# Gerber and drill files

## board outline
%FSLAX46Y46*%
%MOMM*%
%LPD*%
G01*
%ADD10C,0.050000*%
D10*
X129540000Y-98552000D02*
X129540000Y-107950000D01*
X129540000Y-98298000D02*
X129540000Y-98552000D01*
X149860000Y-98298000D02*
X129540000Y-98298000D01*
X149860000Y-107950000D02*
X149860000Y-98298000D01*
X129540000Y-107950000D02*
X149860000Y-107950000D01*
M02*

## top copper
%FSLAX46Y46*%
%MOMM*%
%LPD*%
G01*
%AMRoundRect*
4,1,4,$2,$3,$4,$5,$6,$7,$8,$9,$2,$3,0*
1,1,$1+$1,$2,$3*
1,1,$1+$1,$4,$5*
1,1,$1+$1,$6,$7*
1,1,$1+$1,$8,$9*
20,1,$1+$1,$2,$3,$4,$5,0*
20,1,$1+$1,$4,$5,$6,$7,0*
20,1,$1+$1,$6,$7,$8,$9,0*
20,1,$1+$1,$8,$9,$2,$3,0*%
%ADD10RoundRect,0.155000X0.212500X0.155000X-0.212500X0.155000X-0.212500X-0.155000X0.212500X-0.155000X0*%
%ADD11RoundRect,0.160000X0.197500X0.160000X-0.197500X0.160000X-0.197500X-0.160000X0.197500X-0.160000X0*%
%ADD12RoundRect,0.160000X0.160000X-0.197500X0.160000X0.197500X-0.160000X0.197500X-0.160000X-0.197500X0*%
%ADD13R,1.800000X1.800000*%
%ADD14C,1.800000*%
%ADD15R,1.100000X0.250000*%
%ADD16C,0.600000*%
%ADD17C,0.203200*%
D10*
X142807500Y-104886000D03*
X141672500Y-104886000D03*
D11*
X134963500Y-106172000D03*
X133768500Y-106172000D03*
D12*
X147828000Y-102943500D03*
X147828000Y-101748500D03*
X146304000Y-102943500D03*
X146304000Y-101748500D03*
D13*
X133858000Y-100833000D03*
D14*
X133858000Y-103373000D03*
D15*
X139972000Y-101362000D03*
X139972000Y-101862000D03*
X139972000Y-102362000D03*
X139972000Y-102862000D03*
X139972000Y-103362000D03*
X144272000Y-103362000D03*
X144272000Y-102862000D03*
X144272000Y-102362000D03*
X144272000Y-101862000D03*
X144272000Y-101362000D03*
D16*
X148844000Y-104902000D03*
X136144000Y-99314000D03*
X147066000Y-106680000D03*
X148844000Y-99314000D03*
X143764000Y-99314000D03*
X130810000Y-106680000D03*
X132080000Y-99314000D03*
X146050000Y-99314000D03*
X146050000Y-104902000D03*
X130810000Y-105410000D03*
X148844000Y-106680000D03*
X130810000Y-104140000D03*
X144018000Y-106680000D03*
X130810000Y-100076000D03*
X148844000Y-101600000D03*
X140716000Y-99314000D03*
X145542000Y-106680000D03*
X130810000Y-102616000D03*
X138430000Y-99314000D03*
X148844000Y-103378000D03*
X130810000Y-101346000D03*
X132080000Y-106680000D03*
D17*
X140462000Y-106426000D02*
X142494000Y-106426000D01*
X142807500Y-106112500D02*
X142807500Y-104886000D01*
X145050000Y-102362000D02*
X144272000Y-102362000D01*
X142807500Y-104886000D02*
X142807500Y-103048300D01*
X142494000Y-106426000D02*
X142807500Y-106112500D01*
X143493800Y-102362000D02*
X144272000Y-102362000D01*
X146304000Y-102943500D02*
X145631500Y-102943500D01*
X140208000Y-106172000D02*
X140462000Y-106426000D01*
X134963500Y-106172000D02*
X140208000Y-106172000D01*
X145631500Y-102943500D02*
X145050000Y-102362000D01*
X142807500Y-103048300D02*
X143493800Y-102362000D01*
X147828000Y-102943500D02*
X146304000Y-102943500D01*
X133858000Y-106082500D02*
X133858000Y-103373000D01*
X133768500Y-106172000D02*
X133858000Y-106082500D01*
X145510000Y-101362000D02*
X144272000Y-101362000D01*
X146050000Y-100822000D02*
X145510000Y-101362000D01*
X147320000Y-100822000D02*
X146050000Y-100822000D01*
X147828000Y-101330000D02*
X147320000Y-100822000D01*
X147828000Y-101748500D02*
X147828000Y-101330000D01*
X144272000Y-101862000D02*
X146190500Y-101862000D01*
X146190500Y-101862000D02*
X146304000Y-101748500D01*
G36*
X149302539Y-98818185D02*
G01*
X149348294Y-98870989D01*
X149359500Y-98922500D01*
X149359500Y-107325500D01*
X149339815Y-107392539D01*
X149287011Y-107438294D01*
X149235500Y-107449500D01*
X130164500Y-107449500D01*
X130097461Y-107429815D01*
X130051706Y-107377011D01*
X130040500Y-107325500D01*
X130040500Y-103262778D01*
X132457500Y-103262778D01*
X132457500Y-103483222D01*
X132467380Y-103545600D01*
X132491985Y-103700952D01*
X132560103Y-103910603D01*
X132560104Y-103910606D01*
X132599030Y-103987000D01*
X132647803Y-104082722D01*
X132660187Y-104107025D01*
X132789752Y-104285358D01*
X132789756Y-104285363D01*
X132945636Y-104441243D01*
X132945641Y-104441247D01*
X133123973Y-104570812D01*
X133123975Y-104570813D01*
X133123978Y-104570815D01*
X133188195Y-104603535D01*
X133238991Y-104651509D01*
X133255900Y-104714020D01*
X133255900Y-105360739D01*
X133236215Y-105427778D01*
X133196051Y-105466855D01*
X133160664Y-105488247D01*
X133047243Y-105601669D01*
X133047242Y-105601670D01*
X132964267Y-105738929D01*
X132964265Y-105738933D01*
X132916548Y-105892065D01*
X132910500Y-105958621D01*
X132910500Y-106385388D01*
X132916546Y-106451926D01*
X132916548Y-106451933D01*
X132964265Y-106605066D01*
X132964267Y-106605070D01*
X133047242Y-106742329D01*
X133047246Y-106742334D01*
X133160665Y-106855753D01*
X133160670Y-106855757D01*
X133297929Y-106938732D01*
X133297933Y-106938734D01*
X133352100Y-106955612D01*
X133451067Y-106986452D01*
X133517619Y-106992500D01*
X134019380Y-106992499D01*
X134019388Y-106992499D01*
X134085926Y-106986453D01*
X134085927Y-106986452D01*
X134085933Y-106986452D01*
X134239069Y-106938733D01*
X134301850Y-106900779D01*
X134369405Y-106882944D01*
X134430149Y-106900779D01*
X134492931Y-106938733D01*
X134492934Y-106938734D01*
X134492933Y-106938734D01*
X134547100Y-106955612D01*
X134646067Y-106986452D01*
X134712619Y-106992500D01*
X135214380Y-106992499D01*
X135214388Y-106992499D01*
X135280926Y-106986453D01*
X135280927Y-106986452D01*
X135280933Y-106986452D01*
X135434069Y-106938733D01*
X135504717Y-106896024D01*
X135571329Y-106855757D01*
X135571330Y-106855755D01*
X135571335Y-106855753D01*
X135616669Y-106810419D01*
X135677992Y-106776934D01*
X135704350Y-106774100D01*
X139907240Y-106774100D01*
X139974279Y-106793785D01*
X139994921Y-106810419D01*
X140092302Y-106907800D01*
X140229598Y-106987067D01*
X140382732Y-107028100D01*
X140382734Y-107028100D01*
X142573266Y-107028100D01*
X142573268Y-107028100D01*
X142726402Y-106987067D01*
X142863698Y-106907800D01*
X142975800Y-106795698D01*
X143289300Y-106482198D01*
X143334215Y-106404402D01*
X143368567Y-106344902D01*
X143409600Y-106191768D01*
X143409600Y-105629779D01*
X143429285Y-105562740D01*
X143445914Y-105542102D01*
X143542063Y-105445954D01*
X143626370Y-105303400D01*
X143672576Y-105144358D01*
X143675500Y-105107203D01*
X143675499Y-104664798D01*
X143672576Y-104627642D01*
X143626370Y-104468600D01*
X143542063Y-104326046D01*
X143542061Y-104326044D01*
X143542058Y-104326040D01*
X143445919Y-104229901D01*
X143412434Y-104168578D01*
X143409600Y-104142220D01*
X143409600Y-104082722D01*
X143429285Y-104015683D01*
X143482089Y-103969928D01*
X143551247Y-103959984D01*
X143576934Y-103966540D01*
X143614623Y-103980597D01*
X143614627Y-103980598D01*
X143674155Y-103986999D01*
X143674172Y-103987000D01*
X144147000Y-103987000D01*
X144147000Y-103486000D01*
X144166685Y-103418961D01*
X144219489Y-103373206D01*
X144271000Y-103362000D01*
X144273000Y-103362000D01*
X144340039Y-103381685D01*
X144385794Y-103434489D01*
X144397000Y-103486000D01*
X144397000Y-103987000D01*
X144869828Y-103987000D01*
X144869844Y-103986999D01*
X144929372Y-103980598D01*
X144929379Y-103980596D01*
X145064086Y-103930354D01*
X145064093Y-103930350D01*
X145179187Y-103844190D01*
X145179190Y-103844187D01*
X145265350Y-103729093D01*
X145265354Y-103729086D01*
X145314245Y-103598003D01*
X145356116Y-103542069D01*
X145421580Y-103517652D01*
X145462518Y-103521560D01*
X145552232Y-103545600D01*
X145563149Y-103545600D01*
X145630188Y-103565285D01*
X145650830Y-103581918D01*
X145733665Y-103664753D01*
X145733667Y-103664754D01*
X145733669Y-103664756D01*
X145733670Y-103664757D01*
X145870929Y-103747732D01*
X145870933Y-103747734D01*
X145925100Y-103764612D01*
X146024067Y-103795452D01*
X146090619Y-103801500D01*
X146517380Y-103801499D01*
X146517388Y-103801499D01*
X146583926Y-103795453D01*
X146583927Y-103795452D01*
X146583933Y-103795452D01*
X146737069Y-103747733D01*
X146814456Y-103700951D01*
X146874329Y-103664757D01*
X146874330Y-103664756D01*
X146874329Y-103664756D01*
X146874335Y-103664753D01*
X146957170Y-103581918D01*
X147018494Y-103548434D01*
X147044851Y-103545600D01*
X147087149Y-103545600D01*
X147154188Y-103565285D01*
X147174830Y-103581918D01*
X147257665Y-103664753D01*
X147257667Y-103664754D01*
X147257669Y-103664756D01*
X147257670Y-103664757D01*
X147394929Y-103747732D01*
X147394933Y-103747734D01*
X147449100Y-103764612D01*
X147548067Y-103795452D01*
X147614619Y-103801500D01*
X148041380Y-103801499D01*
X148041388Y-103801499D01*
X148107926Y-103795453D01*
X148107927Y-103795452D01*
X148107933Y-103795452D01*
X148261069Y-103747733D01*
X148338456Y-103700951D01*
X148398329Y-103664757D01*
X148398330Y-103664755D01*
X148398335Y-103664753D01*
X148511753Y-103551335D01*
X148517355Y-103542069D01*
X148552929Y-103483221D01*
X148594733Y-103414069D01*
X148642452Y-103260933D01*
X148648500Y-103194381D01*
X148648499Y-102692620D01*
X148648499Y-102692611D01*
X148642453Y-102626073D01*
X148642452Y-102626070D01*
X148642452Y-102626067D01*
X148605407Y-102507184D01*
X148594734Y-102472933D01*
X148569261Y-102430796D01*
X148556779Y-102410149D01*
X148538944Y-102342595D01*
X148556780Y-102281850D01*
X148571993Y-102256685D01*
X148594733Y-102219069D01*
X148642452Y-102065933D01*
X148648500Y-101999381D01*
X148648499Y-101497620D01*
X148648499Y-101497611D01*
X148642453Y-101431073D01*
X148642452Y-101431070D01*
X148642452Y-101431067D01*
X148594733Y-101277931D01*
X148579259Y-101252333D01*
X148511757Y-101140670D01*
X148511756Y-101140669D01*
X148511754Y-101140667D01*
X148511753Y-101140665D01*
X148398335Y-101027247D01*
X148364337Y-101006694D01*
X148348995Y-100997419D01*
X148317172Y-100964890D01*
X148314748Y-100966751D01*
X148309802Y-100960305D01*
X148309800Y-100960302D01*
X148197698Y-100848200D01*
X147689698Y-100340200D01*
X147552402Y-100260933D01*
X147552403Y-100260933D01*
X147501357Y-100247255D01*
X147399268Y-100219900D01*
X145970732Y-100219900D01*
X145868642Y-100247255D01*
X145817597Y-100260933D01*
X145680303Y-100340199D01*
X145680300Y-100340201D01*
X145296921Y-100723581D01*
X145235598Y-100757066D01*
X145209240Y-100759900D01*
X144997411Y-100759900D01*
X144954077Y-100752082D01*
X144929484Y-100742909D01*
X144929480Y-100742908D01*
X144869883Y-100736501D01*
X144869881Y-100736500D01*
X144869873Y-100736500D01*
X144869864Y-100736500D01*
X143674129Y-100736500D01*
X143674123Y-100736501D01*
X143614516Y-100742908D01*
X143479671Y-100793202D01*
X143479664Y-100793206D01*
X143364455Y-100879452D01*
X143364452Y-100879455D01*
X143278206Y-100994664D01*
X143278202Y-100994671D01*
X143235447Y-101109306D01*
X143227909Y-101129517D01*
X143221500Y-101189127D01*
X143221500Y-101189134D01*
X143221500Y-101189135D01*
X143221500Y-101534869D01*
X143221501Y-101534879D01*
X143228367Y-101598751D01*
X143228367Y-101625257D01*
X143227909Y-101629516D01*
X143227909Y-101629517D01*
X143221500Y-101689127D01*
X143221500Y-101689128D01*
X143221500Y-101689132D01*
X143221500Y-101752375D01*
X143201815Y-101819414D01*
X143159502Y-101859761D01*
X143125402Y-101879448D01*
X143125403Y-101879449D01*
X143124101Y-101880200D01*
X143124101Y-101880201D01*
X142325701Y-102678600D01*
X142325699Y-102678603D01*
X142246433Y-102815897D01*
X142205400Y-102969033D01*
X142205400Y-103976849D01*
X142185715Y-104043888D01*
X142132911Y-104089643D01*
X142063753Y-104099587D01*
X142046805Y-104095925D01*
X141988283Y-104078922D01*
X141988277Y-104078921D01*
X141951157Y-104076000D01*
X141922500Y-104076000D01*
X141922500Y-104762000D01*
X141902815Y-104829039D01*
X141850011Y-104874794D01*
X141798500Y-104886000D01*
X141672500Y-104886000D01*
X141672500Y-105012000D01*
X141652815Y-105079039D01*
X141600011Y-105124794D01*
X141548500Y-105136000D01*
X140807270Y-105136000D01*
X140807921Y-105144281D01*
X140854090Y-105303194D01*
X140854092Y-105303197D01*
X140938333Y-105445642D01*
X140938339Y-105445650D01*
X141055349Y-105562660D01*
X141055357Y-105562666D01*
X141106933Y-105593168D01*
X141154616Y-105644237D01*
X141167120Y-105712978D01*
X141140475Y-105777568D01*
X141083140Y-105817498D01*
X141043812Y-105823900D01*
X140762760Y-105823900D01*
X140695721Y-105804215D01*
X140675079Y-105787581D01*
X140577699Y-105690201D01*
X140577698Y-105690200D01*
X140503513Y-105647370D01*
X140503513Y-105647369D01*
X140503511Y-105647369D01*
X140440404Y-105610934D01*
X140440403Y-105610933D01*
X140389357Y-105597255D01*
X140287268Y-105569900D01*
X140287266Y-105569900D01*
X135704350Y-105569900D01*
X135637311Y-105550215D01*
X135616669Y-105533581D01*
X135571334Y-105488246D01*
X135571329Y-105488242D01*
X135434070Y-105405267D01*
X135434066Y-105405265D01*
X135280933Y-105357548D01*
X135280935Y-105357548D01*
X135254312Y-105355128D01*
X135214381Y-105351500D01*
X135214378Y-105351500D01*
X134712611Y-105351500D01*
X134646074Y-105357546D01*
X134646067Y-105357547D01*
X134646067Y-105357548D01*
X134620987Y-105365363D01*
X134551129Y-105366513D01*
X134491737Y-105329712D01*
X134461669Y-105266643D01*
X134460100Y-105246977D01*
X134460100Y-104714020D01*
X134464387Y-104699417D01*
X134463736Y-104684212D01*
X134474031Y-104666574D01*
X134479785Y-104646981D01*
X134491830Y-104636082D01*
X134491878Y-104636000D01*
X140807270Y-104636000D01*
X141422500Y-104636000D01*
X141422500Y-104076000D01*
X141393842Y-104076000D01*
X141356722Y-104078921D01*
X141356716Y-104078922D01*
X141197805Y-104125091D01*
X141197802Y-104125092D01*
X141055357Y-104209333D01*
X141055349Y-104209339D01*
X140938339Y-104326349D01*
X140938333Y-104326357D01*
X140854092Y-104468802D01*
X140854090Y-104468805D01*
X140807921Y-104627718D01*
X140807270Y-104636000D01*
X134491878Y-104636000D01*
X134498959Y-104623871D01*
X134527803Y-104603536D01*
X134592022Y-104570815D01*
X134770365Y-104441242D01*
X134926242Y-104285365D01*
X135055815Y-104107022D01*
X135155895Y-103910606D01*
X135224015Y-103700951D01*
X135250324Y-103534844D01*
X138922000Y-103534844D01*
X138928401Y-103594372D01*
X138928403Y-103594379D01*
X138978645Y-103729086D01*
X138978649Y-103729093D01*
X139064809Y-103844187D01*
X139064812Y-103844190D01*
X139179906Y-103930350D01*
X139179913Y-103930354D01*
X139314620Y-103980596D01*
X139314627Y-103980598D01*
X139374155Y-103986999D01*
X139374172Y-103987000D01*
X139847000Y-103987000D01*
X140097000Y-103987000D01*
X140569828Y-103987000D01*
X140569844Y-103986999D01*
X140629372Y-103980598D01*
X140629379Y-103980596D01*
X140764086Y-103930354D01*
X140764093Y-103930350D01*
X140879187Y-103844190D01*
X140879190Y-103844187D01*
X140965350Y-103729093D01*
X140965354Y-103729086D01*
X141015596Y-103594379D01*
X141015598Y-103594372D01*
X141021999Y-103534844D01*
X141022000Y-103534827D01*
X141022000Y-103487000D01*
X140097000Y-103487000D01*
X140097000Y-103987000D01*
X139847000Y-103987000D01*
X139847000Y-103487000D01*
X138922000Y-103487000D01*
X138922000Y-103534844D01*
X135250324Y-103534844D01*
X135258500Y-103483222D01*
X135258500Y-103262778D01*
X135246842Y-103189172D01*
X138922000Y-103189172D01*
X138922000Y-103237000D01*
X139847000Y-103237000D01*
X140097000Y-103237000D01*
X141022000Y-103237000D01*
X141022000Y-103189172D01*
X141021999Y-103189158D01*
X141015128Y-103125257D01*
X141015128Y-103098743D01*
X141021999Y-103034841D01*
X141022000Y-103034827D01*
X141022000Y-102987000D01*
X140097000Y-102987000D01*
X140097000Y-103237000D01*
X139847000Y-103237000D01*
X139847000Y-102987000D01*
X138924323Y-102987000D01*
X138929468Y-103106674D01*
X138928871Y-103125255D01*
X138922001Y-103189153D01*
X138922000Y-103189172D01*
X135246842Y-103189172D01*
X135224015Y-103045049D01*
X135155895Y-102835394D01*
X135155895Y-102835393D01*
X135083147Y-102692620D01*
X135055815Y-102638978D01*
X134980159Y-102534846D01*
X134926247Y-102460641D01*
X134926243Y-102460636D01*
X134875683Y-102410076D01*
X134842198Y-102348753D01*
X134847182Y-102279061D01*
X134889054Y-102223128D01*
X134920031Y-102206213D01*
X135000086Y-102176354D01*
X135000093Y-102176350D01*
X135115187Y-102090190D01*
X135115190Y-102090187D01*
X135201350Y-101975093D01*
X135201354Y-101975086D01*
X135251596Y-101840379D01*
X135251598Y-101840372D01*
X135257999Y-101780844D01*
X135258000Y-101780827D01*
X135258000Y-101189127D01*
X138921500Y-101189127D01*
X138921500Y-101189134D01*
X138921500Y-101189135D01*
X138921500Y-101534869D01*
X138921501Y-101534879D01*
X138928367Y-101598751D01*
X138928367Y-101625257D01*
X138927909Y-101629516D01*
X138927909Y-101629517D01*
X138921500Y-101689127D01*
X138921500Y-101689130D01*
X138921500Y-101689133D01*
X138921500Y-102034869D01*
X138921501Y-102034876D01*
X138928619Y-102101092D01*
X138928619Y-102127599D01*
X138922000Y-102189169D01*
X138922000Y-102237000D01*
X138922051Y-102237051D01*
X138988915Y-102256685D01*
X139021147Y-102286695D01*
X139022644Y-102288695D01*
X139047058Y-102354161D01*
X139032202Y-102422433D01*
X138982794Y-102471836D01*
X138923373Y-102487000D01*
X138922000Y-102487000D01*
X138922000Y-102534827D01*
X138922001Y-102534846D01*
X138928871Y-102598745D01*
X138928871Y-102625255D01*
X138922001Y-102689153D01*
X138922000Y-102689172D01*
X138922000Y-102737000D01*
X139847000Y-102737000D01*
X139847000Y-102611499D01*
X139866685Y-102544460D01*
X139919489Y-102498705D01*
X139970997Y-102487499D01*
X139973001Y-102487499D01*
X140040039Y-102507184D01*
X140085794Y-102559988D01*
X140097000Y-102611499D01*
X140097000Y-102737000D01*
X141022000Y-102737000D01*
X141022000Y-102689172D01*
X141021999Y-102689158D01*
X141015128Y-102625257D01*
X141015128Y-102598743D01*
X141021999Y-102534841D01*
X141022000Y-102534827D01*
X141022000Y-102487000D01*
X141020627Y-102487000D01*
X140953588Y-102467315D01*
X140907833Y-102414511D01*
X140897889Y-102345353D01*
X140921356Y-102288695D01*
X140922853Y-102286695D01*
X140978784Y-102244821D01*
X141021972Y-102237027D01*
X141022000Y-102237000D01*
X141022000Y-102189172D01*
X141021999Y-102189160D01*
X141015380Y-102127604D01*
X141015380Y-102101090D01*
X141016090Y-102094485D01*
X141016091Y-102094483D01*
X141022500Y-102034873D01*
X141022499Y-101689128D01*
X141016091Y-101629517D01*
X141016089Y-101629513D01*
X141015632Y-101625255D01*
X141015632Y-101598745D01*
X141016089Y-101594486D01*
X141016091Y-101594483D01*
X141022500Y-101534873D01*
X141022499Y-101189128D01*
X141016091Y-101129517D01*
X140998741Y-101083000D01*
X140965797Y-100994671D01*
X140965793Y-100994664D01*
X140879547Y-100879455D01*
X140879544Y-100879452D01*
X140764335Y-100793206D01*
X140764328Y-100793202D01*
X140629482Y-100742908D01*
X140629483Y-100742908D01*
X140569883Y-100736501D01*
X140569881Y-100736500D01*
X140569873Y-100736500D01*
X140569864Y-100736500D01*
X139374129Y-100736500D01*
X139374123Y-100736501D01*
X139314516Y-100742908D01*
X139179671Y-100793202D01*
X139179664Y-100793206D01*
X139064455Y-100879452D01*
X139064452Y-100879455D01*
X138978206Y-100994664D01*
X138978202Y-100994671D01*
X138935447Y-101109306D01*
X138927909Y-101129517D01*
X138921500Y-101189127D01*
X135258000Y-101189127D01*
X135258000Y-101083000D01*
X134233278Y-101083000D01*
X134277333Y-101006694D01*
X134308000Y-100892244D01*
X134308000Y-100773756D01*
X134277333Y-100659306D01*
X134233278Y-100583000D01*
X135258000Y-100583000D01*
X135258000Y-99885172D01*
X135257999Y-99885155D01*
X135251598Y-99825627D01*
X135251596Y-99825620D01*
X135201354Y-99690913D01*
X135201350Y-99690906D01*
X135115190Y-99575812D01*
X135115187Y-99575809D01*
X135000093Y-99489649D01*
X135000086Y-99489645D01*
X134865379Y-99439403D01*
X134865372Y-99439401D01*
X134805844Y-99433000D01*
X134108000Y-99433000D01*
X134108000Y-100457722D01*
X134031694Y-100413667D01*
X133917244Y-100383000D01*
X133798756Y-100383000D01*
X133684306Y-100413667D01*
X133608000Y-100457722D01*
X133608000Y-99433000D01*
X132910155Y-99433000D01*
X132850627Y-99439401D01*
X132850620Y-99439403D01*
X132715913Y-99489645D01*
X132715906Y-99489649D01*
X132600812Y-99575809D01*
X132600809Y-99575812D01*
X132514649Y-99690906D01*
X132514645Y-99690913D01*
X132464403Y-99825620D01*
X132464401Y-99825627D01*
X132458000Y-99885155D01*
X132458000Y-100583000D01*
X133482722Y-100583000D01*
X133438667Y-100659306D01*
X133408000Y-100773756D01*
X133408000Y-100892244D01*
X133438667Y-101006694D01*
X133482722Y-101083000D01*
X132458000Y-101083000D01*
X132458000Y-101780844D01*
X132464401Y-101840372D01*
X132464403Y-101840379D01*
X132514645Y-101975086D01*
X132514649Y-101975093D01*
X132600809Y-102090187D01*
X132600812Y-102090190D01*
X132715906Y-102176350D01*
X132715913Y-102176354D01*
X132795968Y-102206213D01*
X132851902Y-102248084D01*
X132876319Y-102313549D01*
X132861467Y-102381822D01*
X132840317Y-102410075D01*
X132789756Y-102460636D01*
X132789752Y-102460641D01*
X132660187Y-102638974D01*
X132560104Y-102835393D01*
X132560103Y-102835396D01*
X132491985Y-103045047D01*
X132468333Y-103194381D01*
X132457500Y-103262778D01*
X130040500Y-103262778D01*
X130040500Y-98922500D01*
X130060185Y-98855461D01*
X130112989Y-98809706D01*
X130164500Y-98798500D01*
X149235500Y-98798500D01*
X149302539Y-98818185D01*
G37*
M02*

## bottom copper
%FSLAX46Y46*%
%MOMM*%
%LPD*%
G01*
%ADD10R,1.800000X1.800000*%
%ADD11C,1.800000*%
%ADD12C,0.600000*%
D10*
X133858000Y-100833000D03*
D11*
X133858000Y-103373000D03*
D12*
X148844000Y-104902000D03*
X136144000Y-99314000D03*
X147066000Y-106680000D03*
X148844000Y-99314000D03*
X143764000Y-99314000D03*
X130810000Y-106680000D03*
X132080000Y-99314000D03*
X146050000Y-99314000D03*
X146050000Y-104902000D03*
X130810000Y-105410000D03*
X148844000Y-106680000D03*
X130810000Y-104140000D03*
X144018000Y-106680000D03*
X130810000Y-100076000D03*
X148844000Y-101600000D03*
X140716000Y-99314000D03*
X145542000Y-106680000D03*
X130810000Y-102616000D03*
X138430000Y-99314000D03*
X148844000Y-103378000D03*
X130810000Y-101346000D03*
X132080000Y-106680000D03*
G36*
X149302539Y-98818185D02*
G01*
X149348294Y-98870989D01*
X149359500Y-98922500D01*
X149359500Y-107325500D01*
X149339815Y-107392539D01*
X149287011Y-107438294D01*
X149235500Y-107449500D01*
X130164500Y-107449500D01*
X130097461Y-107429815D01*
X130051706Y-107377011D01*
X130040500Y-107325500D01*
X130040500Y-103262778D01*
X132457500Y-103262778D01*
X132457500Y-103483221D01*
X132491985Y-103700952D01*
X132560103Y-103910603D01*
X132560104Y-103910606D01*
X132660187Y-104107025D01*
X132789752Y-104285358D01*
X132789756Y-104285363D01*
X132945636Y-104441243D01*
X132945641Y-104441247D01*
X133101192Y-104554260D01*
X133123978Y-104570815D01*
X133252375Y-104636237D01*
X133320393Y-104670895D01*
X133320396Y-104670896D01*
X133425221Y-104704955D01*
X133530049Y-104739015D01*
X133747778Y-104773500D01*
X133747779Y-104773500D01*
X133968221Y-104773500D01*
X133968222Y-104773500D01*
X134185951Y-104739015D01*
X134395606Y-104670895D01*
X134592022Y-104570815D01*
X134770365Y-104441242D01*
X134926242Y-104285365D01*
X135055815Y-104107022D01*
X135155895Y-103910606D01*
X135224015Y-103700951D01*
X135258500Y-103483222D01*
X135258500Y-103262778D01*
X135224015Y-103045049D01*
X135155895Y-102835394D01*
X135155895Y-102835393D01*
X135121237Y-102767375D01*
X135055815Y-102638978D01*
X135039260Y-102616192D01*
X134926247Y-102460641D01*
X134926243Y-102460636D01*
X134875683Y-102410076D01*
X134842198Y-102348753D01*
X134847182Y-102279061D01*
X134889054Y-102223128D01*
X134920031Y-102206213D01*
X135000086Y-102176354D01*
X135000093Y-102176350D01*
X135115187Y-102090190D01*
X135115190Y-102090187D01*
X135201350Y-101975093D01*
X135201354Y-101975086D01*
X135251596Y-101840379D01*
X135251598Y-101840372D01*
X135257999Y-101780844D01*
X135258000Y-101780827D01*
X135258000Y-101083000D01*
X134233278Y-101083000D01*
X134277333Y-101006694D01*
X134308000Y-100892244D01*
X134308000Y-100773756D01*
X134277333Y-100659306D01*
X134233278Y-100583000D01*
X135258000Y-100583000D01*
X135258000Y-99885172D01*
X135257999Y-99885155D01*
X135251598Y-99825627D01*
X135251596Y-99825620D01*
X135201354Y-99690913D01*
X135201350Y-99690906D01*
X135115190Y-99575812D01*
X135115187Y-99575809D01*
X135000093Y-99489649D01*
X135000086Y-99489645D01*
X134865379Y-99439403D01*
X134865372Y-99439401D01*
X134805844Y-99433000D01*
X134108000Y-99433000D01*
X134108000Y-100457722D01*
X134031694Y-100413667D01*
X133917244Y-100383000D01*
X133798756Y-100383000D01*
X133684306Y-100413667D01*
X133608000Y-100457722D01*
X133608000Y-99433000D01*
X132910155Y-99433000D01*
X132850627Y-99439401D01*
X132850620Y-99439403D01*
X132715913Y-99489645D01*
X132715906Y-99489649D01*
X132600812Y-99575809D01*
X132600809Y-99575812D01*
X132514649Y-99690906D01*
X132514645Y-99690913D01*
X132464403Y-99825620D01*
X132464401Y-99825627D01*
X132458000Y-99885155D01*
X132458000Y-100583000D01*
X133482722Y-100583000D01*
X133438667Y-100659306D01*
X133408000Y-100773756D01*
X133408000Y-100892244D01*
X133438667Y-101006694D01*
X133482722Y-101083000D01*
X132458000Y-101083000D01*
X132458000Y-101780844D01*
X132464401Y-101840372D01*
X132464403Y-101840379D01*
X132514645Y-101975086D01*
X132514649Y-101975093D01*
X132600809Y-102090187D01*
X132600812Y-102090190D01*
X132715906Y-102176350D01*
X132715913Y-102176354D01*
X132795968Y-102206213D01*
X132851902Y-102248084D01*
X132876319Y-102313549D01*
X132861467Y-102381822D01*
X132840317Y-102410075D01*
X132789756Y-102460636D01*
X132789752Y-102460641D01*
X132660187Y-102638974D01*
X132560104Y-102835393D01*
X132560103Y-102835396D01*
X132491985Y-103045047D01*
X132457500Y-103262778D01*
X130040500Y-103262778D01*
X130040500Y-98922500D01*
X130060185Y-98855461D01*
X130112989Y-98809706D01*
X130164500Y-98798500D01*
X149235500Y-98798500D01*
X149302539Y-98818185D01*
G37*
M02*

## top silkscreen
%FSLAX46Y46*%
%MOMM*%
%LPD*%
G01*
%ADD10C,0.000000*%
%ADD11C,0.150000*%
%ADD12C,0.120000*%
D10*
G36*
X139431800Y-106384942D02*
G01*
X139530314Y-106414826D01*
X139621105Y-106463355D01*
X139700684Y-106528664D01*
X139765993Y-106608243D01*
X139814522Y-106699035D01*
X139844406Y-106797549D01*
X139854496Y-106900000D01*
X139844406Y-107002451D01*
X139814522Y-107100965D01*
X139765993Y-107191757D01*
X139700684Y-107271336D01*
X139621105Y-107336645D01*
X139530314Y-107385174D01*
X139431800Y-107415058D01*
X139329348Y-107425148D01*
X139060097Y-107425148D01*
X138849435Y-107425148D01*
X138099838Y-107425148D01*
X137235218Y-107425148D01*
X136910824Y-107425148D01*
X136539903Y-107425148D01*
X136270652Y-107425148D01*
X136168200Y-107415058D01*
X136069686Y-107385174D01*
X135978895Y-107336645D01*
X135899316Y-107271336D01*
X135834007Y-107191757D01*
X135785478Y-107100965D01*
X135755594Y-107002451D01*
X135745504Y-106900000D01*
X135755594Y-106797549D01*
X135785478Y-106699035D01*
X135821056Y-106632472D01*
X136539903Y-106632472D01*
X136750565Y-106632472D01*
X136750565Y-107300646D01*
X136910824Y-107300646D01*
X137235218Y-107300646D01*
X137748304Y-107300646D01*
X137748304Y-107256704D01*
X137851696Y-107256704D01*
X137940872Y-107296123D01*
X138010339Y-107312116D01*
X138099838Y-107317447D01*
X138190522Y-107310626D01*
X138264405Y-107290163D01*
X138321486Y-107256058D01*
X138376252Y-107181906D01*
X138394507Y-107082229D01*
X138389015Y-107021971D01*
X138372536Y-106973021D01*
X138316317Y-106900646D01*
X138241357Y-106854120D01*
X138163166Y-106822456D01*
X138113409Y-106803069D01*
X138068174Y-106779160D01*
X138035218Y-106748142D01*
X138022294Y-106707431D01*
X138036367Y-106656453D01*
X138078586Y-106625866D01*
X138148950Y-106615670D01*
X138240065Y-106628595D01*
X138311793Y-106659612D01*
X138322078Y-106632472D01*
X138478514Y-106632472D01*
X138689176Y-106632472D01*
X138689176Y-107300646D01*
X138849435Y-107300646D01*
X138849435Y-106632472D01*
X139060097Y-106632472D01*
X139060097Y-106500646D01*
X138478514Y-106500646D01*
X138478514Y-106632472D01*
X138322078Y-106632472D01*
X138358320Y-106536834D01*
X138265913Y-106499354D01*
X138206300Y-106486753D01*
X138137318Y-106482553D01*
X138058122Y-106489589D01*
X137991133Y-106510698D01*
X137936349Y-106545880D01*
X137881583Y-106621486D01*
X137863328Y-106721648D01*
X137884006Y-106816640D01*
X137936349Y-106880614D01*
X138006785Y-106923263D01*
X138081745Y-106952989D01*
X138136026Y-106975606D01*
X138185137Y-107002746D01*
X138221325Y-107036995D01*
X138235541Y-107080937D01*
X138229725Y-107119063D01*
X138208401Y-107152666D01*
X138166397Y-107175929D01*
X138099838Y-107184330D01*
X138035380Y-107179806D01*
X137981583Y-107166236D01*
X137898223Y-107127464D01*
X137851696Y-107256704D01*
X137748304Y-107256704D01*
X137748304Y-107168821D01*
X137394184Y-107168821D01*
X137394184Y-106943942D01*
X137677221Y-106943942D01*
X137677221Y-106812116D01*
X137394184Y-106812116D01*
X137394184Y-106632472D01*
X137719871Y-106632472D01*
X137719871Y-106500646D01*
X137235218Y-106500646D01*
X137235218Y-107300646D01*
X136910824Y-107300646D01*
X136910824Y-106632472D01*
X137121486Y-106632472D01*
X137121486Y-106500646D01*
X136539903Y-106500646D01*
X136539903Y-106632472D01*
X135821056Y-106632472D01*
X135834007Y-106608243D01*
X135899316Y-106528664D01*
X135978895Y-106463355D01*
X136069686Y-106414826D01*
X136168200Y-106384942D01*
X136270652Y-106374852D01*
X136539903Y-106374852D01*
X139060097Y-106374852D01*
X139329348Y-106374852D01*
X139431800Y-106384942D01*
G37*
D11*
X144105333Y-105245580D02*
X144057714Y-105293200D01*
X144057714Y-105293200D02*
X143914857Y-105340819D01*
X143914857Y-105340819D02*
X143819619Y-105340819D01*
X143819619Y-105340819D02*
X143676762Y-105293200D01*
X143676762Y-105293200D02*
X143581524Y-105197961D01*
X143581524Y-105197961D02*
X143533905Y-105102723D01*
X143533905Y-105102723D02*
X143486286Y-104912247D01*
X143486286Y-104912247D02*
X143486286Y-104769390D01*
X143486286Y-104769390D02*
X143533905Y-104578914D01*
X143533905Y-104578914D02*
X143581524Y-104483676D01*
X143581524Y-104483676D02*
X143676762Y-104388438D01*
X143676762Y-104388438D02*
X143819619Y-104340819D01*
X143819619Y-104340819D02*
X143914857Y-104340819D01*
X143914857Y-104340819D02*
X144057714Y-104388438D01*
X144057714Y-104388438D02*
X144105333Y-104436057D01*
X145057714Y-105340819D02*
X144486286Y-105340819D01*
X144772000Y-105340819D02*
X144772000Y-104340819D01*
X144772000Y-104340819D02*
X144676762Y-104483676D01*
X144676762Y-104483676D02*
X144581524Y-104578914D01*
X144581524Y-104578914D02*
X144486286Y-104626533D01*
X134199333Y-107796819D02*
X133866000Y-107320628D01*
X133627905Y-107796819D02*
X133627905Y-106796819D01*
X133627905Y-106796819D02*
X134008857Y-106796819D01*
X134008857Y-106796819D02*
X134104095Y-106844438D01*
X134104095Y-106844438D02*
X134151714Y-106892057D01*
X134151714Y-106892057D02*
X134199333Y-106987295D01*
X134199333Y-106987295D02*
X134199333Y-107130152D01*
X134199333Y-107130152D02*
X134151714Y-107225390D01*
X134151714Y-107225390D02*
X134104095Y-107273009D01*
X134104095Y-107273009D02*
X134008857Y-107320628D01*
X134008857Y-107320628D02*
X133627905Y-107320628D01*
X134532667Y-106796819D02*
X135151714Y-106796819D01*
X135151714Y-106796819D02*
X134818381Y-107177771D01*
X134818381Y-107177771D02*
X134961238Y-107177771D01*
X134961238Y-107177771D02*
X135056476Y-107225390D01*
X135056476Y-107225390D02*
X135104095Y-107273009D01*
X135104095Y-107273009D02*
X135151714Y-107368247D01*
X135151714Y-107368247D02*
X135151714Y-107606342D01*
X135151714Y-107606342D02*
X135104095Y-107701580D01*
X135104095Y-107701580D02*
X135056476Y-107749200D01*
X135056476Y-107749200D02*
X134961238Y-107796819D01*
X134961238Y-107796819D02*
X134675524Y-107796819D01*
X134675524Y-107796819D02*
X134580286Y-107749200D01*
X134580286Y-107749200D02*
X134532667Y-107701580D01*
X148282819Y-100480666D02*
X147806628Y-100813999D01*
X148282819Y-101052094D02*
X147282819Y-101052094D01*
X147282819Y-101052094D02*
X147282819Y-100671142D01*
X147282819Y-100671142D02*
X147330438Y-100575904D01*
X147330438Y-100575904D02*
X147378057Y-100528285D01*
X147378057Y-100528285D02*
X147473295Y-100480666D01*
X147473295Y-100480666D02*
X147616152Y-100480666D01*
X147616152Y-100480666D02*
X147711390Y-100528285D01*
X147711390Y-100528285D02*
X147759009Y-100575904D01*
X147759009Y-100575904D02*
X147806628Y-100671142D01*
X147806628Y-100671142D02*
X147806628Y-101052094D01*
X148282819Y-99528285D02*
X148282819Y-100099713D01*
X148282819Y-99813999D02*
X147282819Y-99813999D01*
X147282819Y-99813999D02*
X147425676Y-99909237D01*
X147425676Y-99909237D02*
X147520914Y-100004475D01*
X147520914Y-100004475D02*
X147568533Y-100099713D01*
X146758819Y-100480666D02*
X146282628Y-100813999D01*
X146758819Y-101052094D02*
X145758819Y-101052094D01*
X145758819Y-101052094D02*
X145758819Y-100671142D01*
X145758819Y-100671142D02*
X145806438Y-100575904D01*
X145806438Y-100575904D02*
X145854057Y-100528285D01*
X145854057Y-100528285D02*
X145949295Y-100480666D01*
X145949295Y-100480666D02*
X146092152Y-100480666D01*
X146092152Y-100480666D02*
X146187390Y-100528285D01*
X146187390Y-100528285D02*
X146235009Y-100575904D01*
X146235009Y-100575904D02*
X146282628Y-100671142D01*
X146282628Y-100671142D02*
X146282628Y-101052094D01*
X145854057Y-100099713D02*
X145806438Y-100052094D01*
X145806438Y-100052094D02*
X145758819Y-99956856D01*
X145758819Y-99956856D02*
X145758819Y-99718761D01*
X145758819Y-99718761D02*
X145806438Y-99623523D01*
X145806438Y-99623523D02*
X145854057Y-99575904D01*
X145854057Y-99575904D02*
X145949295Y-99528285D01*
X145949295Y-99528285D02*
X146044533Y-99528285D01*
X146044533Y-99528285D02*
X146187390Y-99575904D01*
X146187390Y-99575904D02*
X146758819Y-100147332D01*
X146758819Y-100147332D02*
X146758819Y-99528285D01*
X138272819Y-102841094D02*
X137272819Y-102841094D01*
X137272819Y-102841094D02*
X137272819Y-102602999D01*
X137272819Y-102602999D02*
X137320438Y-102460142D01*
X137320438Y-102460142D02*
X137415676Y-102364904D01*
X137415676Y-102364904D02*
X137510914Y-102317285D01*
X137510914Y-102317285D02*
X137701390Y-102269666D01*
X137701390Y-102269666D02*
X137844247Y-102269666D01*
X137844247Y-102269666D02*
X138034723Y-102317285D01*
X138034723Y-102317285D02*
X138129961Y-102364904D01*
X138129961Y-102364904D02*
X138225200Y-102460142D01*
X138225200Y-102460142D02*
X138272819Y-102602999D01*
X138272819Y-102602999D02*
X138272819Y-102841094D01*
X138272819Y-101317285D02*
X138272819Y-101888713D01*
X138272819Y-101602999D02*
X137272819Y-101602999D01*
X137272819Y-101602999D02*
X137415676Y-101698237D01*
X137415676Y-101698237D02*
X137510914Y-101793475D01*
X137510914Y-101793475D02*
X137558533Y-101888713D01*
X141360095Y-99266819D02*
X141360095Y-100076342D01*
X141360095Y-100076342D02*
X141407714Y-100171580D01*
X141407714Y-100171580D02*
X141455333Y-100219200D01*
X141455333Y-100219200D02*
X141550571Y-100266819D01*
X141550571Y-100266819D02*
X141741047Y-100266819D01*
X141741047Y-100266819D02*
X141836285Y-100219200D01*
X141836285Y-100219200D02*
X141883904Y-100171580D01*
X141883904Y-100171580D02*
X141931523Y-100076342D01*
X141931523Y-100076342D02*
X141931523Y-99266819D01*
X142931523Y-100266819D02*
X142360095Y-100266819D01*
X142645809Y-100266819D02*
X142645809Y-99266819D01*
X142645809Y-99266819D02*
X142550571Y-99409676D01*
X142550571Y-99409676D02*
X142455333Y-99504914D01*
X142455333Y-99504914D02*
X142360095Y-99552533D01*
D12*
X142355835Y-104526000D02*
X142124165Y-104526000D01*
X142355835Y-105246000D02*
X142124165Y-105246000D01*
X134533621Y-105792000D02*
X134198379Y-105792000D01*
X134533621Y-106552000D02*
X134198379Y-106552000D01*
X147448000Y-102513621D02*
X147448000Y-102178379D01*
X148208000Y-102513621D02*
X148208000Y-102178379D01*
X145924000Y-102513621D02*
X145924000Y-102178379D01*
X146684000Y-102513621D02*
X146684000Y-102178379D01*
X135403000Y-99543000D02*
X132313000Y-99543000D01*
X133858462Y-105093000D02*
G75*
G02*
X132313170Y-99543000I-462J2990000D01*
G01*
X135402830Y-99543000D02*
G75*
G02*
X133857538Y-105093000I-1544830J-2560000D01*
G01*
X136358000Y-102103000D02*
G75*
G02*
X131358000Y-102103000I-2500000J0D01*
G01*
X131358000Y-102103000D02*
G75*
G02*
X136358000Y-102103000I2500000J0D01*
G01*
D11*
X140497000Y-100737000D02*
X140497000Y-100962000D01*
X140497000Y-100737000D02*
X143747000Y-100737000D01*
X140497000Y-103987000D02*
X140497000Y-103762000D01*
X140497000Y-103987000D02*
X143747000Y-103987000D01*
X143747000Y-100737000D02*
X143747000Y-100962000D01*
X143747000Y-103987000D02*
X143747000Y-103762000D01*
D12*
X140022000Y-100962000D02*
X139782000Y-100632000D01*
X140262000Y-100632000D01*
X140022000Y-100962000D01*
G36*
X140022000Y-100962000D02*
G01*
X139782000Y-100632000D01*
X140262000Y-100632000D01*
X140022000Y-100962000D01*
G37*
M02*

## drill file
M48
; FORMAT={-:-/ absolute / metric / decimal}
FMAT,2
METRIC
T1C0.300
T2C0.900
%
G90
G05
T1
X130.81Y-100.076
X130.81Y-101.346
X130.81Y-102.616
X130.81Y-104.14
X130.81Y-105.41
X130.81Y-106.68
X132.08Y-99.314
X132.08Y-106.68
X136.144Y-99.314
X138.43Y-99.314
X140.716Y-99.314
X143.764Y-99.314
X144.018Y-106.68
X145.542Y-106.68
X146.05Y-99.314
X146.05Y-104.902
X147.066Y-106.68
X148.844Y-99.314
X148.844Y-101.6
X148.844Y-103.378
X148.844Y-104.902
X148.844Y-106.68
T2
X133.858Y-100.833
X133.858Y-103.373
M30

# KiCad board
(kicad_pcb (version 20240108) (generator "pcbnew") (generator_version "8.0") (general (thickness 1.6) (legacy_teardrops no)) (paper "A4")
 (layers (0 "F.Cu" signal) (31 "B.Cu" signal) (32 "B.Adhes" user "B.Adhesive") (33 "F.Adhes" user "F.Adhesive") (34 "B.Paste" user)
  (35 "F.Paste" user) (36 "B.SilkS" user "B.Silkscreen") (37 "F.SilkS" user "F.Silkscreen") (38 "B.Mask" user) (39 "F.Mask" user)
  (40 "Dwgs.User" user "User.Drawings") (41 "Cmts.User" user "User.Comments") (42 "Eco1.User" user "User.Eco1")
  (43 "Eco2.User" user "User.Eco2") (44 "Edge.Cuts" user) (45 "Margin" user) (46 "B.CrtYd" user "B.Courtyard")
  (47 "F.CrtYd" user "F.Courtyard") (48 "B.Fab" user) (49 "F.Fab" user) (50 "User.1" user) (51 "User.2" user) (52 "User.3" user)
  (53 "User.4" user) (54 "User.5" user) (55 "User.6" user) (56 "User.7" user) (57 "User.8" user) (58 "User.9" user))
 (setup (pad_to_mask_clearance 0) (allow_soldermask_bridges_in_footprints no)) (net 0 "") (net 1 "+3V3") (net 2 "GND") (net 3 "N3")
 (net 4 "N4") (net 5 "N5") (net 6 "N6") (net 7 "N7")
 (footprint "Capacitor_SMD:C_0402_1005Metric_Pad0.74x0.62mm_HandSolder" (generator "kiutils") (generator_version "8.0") (layer "F.Cu")
  (at 142.24 104.886 180)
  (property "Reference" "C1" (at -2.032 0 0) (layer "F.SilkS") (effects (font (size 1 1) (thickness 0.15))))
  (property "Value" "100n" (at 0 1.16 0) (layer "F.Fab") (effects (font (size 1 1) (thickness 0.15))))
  (fp_line (start -0.115835 0.36) (end 0.115835 0.36) (stroke (width 0.12) (type solid)) (layer "F.SilkS"))
  (fp_line (start -0.115835 -0.36) (end 0.115835 -0.36) (stroke (width 0.12) (type solid)) (layer "F.SilkS"))
  (pad "1" smd roundrect (at -0.5675 0 180) (size 0.735 0.62) (layers "F.Cu" "F.Paste" "F.Mask") (roundrect_rratio 0.25) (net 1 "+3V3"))
  (pad "2" smd roundrect (at 0.5675 0 180) (size 0.735 0.62) (layers "F.Cu" "F.Paste" "F.Mask") (roundrect_rratio 0.25) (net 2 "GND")))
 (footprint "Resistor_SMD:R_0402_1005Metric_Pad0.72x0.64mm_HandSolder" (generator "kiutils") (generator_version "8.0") (layer "F.Cu")
  (at 134.366 106.172 180)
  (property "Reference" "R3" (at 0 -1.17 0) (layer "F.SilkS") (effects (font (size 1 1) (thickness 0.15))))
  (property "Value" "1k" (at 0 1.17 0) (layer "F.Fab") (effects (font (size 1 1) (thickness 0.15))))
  (fp_line (start -0.167621 0.38) (end 0.167621 0.38) (stroke (width 0.12) (type solid)) (layer "F.SilkS"))
  (fp_line (start -0.167621 -0.38) (end 0.167621 -0.38) (stroke (width 0.12) (type solid)) (layer "F.SilkS"))
  (pad "1" smd roundrect (at -0.5975 0 180) (size 0.715 0.64) (layers "F.Cu" "F.Paste" "F.Mask") (roundrect_rratio 0.25) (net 1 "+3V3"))
  (pad "2" smd roundrect (at 0.5975 0 180) (size 0.715 0.64) (layers "F.Cu" "F.Paste" "F.Mask") (roundrect_rratio 0.25) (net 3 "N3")))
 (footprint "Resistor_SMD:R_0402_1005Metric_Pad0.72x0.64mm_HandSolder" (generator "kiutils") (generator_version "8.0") (layer "F.Cu")
  (at 147.828 102.346 90)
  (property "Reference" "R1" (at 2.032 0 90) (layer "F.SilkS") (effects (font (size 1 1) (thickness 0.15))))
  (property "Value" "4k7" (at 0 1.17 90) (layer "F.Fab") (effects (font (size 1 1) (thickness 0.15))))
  (fp_line (start -0.167621 -0.38) (end 0.167621 -0.38) (stroke (width 0.12) (type solid)) (layer "F.SilkS"))
  (fp_line (start -0.167621 0.38) (end 0.167621 0.38) (stroke (width 0.12) (type solid)) (layer "F.SilkS"))
  (pad "1" smd roundrect (at -0.5975 0 90) (size 0.715 0.64) (layers "F.Cu" "F.Paste" "F.Mask") (roundrect_rratio 0.25) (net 1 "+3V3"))
  (pad "2" smd roundrect (at 0.5975 0 90) (size 0.715 0.64) (layers "F.Cu" "F.Paste" "F.Mask") (roundrect_rratio 0.25) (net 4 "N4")))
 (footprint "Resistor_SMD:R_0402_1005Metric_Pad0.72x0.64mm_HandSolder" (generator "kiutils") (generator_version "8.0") (layer "F.Cu")
  (at 146.304 102.346 90)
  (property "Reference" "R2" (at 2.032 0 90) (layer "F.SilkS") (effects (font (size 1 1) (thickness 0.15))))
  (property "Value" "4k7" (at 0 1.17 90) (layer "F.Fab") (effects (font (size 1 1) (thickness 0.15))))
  (fp_line (start -0.167621 -0.38) (end 0.167621 -0.38) (stroke (width 0.12) (type solid)) (layer "F.SilkS"))
  (fp_line (start -0.167621 0.38) (end 0.167621 0.38) (stroke (width 0.12) (type solid)) (layer "F.SilkS"))
  (pad "1" smd roundrect (at -0.5975 0 90) (size 0.715 0.64) (layers "F.Cu" "F.Paste" "F.Mask") (roundrect_rratio 0.25) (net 1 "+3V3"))
  (pad "2" smd roundrect (at 0.5975 0 90) (size 0.715 0.64) (layers "F.Cu" "F.Paste" "F.Mask") (roundrect_rratio 0.25) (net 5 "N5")))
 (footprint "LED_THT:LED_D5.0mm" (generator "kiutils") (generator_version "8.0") (layer "F.Cu") (at 133.858 100.833 -90)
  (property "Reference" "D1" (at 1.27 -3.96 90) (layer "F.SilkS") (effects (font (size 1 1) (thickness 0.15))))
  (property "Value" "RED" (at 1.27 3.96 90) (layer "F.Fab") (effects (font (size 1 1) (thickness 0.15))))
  (fp_line (start -1.29 -1.545) (end -1.29 1.545) (stroke (width 0.12) (type solid)) (layer "F.SilkS"))
  (fp_arc (start 4.26 -0.000462) (mid 2.072002 2.880433) (end -1.29 1.54483) (stroke (width 0.12) (type solid)) (layer "F.SilkS"))
  (fp_arc (start -1.29 -1.54483) (mid 2.072002 -2.880433) (end 4.26 0.000462) (stroke (width 0.12) (type solid)) (layer "F.SilkS"))
  (fp_circle (center 1.27 0) (end 3.77 0) (stroke (width 0.12) (type solid)) (fill none) (layer "F.SilkS"))
  (pad "1" thru_hole rect (at 0 0 270) (size 1.8 1.8) (drill 0.9) (layers "*.Cu" "*.Mask") (remove_unused_layers no) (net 2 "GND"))
  (pad "2" thru_hole circle (at 2.54 0 270) (size 1.8 1.8) (drill 0.9) (layers "*.Cu" "*.Mask") (remove_unused_layers no) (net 3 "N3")))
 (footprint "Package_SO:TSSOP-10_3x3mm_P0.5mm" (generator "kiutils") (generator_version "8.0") (layer "F.Cu") (at 142.122 102.362)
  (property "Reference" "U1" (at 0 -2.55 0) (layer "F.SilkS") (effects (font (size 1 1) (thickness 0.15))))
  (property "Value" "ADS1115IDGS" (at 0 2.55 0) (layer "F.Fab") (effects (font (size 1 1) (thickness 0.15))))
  (fp_line (start -1.625 -1.625) (end -1.625 -1.4) (stroke (width 0.15) (type solid)) (layer "F.SilkS"))
  (fp_line (start -1.625 -1.625) (end 1.625 -1.625) (stroke (width 0.15) (type solid)) (layer "F.SilkS"))
  (fp_line (start -1.625 1.625) (end -1.625 1.4) (stroke (width 0.15) (type solid)) (layer "F.SilkS"))
  (fp_line (start -1.625 1.625) (end 1.625 1.625) (stroke (width 0.15) (type solid)) (layer "F.SilkS"))
  (fp_line (start 1.625 -1.625) (end 1.625 -1.4) (stroke (width 0.15) (type solid)) (layer "F.SilkS"))
  (fp_line (start 1.625 1.625) (end 1.625 1.4) (stroke (width 0.15) (type solid)) (layer "F.SilkS"))
  (fp_poly
   (pts (xy -2.1 -1.4) (xy -2.34 -1.73) (xy -1.86 -1.73) (xy -2.1 -1.4)) (stroke (width 0.12) (type solid)) (fill solid) (layer "F.SilkS"))
  (pad "1" smd rect (at -2.15 -1) (size 1.1 0.25) (layers "F.Cu" "F.Paste" "F.Mask") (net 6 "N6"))
  (pad "2" smd rect (at -2.15 -0.5) (size 1.1 0.25) (layers "F.Cu" "F.Paste" "F.Mask") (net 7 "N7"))
  (pad "3" smd rect (at -2.15 0) (size 1.1 0.25) (layers "F.Cu" "F.Paste" "F.Mask") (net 2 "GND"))
  (pad "4" smd rect (at -2.15 0.5) (size 1.1 0.25) (layers "F.Cu" "F.Paste" "F.Mask") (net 2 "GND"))
  (pad "5" smd rect (at -2.15 1) (size 1.1 0.25) (layers "F.Cu" "F.Paste" "F.Mask") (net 2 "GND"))
  (pad "6" smd rect (at 2.15 1) (size 1.1 0.25) (layers "F.Cu" "F.Paste" "F.Mask") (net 2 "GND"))
  (pad "7" smd rect (at 2.15 0.5) (size 1.1 0.25) (layers "F.Cu" "F.Paste" "F.Mask") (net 2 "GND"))
  (pad "8" smd rect (at 2.15 0) (size 1.1 0.25) (layers "F.Cu" "F.Paste" "F.Mask") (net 1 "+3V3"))
  (pad "9" smd rect (at 2.15 -0.5) (size 1.1 0.25) (layers "F.Cu" "F.Paste" "F.Mask") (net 5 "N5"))
  (pad "10" smd rect (at 2.15 -1) (size 1.1 0.25) (layers "F.Cu" "F.Paste" "F.Mask") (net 4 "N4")))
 (gr_line (start 129.54 98.552) (end 129.54 107.95) (stroke (width 0.05) (type default)) (layer "Edge.Cuts"))
 (gr_line (start 129.54 98.298) (end 129.54 98.552) (stroke (width 0.05) (type default)) (layer "Edge.Cuts"))
 (gr_line (start 149.86 98.298) (end 129.54 98.298) (stroke (width 0.05) (type default)) (layer "Edge.Cuts"))
 (gr_line (start 149.86 107.95) (end 149.86 98.298) (stroke (width 0.05) (type default)) (layer "Edge.Cuts"))
 (gr_line (start 129.54 107.95) (end 149.86 107.95) (stroke (width 0.05) (type default)) (layer "Edge.Cuts"))
 (gr_poly
  (pts (xy 136.539903 106.374852) (xy 136.270652 106.374852) (xy 136.1682 106.384942) (xy 136.069686 106.414826) (xy 135.978895 106.463355)
   (xy 135.899316 106.528664) (xy 135.834007 106.608243) (xy 135.785478 106.699035) (xy 135.755594 106.797549) (xy 135.745504 106.9)
   (xy 135.755594 107.002451) (xy 135.785478 107.100965) (xy 135.834007 107.191757) (xy 135.899316 107.271336) (xy 135.978895 107.336645)
   (xy 136.069686 107.385174) (xy 136.1682 107.415058) (xy 136.270652 107.425148) (xy 136.539903 107.425148) (xy 136.910824 107.425148)
   (xy 136.910824 107.300646) (xy 136.750565 107.300646) (xy 136.750565 106.632472) (xy 136.539903 106.632472) (xy 136.539903 106.500646)
   (xy 137.121486 106.500646) (xy 137.121486 106.632472) (xy 136.910824 106.632472) (xy 136.910824 107.300646) (xy 136.910824 107.425148)
   (xy 137.235218 107.425148) (xy 137.235218 107.300646) (xy 137.235218 106.500646) (xy 137.719871 106.500646) (xy 137.719871 106.632472)
   (xy 137.394184 106.632472) (xy 137.394184 106.812116) (xy 137.677221 106.812116) (xy 137.677221 106.943942) (xy 137.394184 106.943942)
   (xy 137.394184 107.168821) (xy 137.748304 107.168821) (xy 137.748304 107.300646) (xy 137.235218 107.300646) (xy 137.235218 107.425148)
   (xy 138.099838 107.425148) (xy 138.099838 107.317447) (xy 138.010339 107.312116) (xy 137.940872 107.296123) (xy 137.851696 107.256704)
   (xy 137.898223 107.127464) (xy 137.981583 107.166236) (xy 138.03538 107.179806) (xy 138.099838 107.18433) (xy 138.166397 107.175929)
   (xy 138.208401 107.152666) (xy 138.229725 107.119063) (xy 138.235541 107.080937) (xy 138.221325 107.036995) (xy 138.185137 107.002746)
   (xy 138.136026 106.975606) (xy 138.081745 106.952989) (xy 138.006785 106.923263) (xy 137.936349 106.880614) (xy 137.884006 106.81664)
   (xy 137.863328 106.721648) (xy 137.881583 106.621486) (xy 137.936349 106.54588) (xy 137.991133 106.510698) (xy 138.058122 106.489589)
   (xy 138.137318 106.482553) (xy 138.2063 106.486753) (xy 138.265913 106.499354) (xy 138.35832 106.536834) (xy 138.311793 106.659612)
   (xy 138.240065 106.628595) (xy 138.14895 106.61567) (xy 138.078586 106.625866) (xy 138.036367 106.656453) (xy 138.022294 106.707431)
   (xy 138.035218 106.748142) (xy 138.068174 106.77916) (xy 138.113409 106.803069) (xy 138.163166 106.822456) (xy 138.241357 106.85412)
   (xy 138.316317 106.900646) (xy 138.372536 106.973021) (xy 138.389015 107.021971) (xy 138.394507 107.082229) (xy 138.376252 107.181906)
   (xy 138.321486 107.256058) (xy 138.264405 107.290163) (xy 138.190522 107.310626) (xy 138.099838 107.317447) (xy 138.099838 107.425148)
   (xy 138.849435 107.425148) (xy 138.849435 107.300646) (xy 138.689176 107.300646) (xy 138.689176 106.632472) (xy 138.478514 106.632472)
   (xy 138.478514 106.500646) (xy 139.060097 106.500646) (xy 139.060097 106.632472) (xy 138.849435 106.632472) (xy 138.849435 107.300646)
   (xy 138.849435 107.425148) (xy 139.060097 107.425148) (xy 139.329348 107.425148) (xy 139.4318 107.415058) (xy 139.530314 107.385174)
   (xy 139.621105 107.336645) (xy 139.700684 107.271336) (xy 139.765993 107.191757) (xy 139.814522 107.100965) (xy 139.844406 107.002451)
   (xy 139.854496 106.9) (xy 139.844406 106.797549) (xy 139.814522 106.699035) (xy 139.765993 106.608243) (xy 139.700684 106.528664)
   (xy 139.621105 106.463355) (xy 139.530314 106.414826) (xy 139.4318 106.384942) (xy 139.329348 106.374852) (xy 139.060097 106.374852)
   (xy 136.539903 106.374852))
  (layer "F.SilkS") (width 0) (fill solid))
 (segment (start 140.462 106.426) (end 142.494 106.426) (width 0.2032) (layer "F.Cu") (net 1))
 (segment (start 142.8075 106.1125) (end 142.8075 104.886) (width 0.2032) (layer "F.Cu") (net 1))
 (segment (start 145.05 102.362) (end 144.272 102.362) (width 0.2032) (layer "F.Cu") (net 1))
 (segment (start 142.8075 104.886) (end 142.8075 103.0483) (width 0.2032) (layer "F.Cu") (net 1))
 (segment (start 142.494 106.426) (end 142.8075 106.1125) (width 0.2032) (layer "F.Cu") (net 1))
 (segment (start 143.4938 102.362) (end 144.272 102.362) (width 0.2032) (layer "F.Cu") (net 1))
 (segment (start 146.304 102.9435) (end 145.6315 102.9435) (width 0.2032) (layer "F.Cu") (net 1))
 (segment (start 140.208 106.172) (end 140.462 106.426) (width 0.2032) (layer "F.Cu") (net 1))
 (segment (start 134.9635 106.172) (end 140.208 106.172) (width 0.2032) (layer "F.Cu") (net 1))
 (segment (start 145.6315 102.9435) (end 145.05 102.362) (width 0.2032) (layer "F.Cu") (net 1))
 (segment (start 142.8075 103.0483) (end 143.4938 102.362) (width 0.2032) (layer "F.Cu") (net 1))
 (segment (start 147.828 102.9435) (end 146.304 102.9435) (width 0.2032) (layer "F.Cu") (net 1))
 (via (at 148.844 104.902) (size 0.6) (drill 0.3) (layers "F.Cu" "B.Cu") (free yes) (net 2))
 (via (at 136.144 99.314) (size 0.6) (drill 0.3) (layers "F.Cu" "B.Cu") (free yes) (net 2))
 (via (at 147.066 106.68) (size 0.6) (drill 0.3) (layers "F.Cu" "B.Cu") (free yes) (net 2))
 (via (at 148.844 99.314) (size 0.6) (drill 0.3) (layers "F.Cu" "B.Cu") (free yes) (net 2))
 (via (at 143.764 99.314) (size 0.6) (drill 0.3) (layers "F.Cu" "B.Cu") (free yes) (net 2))
 (via (at 130.81 106.68) (size 0.6) (drill 0.3) (layers "F.Cu" "B.Cu") (free yes) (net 2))
 (via (at 132.08 99.314) (size 0.6) (drill 0.3) (layers "F.Cu" "B.Cu") (free yes) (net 2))
 (via (at 146.05 99.314) (size 0.6) (drill 0.3) (layers "F.Cu" "B.Cu") (free yes) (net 2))
 (via (at 146.05 104.902) (size 0.6) (drill 0.3) (layers "F.Cu" "B.Cu") (free yes) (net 2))
 (via (at 130.81 105.41) (size 0.6) (drill 0.3) (layers "F.Cu" "B.Cu") (free yes) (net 2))
 (via (at 148.844 106.68) (size 0.6) (drill 0.3) (layers "F.Cu" "B.Cu") (free yes) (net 2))
 (via (at 130.81 104.14) (size 0.6) (drill 0.3) (layers "F.Cu" "B.Cu") (free yes) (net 2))
 (via (at 144.018 106.68) (size 0.6) (drill 0.3) (layers "F.Cu" "B.Cu") (free yes) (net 2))
 (via (at 130.81 100.076) (size 0.6) (drill 0.3) (layers "F.Cu" "B.Cu") (free yes) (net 2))
 (via (at 148.844 101.6) (size 0.6) (drill 0.3) (layers "F.Cu" "B.Cu") (free yes) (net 2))
 (via (at 140.716 99.314) (size 0.6) (drill 0.3) (layers "F.Cu" "B.Cu") (free yes) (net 2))
 (via (at 145.542 106.68) (size 0.6) (drill 0.3) (layers "F.Cu" "B.Cu") (free yes) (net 2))
 (via (at 130.81 102.616) (size 0.6) (drill 0.3) (layers "F.Cu" "B.Cu") (free yes) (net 2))
 (via (at 138.43 99.314) (size 0.6) (drill 0.3) (layers "F.Cu" "B.Cu") (free yes) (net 2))
 (via (at 148.844 103.378) (size 0.6) (drill 0.3) (layers "F.Cu" "B.Cu") (free yes) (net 2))
 (via (at 130.81 101.346) (size 0.6) (drill 0.3) (layers "F.Cu" "B.Cu") (free yes) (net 2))
 (via (at 132.08 106.68) (size 0.6) (drill 0.3) (layers "F.Cu" "B.Cu") (free yes) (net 2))
 (segment (start 133.858 106.0825) (end 133.858 103.373) (width 0.2032) (layer "F.Cu") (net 3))
 (segment (start 133.7685 106.172) (end 133.858 106.0825) (width 0.2032) (layer "F.Cu") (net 3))
 (segment (start 145.51 101.362) (end 144.272 101.362) (width 0.2032) (layer "F.Cu") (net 4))
 (segment (start 146.05 100.822) (end 145.51 101.362) (width 0.2032) (layer "F.Cu") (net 4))
 (segment (start 147.32 100.822) (end 146.05 100.822) (width 0.2032) (layer "F.Cu") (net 4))
 (segment (start 147.828 101.33) (end 147.32 100.822) (width 0.2032) (layer "F.Cu") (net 4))
 (segment (start 147.828 101.7485) (end 147.828 101.33) (width 0.2032) (layer "F.Cu") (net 4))
 (segment (start 144.272 101.862) (end 146.1905 101.862) (width 0.2032) (layer "F.Cu") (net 5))
 (segment (start 146.1905 101.862) (end 146.304 101.7485) (width 0.2032) (layer "F.Cu") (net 5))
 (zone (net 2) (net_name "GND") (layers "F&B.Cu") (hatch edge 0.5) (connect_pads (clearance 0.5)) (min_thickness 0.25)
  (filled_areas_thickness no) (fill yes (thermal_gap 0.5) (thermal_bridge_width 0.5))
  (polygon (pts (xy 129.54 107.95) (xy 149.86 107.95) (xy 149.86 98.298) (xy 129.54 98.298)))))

